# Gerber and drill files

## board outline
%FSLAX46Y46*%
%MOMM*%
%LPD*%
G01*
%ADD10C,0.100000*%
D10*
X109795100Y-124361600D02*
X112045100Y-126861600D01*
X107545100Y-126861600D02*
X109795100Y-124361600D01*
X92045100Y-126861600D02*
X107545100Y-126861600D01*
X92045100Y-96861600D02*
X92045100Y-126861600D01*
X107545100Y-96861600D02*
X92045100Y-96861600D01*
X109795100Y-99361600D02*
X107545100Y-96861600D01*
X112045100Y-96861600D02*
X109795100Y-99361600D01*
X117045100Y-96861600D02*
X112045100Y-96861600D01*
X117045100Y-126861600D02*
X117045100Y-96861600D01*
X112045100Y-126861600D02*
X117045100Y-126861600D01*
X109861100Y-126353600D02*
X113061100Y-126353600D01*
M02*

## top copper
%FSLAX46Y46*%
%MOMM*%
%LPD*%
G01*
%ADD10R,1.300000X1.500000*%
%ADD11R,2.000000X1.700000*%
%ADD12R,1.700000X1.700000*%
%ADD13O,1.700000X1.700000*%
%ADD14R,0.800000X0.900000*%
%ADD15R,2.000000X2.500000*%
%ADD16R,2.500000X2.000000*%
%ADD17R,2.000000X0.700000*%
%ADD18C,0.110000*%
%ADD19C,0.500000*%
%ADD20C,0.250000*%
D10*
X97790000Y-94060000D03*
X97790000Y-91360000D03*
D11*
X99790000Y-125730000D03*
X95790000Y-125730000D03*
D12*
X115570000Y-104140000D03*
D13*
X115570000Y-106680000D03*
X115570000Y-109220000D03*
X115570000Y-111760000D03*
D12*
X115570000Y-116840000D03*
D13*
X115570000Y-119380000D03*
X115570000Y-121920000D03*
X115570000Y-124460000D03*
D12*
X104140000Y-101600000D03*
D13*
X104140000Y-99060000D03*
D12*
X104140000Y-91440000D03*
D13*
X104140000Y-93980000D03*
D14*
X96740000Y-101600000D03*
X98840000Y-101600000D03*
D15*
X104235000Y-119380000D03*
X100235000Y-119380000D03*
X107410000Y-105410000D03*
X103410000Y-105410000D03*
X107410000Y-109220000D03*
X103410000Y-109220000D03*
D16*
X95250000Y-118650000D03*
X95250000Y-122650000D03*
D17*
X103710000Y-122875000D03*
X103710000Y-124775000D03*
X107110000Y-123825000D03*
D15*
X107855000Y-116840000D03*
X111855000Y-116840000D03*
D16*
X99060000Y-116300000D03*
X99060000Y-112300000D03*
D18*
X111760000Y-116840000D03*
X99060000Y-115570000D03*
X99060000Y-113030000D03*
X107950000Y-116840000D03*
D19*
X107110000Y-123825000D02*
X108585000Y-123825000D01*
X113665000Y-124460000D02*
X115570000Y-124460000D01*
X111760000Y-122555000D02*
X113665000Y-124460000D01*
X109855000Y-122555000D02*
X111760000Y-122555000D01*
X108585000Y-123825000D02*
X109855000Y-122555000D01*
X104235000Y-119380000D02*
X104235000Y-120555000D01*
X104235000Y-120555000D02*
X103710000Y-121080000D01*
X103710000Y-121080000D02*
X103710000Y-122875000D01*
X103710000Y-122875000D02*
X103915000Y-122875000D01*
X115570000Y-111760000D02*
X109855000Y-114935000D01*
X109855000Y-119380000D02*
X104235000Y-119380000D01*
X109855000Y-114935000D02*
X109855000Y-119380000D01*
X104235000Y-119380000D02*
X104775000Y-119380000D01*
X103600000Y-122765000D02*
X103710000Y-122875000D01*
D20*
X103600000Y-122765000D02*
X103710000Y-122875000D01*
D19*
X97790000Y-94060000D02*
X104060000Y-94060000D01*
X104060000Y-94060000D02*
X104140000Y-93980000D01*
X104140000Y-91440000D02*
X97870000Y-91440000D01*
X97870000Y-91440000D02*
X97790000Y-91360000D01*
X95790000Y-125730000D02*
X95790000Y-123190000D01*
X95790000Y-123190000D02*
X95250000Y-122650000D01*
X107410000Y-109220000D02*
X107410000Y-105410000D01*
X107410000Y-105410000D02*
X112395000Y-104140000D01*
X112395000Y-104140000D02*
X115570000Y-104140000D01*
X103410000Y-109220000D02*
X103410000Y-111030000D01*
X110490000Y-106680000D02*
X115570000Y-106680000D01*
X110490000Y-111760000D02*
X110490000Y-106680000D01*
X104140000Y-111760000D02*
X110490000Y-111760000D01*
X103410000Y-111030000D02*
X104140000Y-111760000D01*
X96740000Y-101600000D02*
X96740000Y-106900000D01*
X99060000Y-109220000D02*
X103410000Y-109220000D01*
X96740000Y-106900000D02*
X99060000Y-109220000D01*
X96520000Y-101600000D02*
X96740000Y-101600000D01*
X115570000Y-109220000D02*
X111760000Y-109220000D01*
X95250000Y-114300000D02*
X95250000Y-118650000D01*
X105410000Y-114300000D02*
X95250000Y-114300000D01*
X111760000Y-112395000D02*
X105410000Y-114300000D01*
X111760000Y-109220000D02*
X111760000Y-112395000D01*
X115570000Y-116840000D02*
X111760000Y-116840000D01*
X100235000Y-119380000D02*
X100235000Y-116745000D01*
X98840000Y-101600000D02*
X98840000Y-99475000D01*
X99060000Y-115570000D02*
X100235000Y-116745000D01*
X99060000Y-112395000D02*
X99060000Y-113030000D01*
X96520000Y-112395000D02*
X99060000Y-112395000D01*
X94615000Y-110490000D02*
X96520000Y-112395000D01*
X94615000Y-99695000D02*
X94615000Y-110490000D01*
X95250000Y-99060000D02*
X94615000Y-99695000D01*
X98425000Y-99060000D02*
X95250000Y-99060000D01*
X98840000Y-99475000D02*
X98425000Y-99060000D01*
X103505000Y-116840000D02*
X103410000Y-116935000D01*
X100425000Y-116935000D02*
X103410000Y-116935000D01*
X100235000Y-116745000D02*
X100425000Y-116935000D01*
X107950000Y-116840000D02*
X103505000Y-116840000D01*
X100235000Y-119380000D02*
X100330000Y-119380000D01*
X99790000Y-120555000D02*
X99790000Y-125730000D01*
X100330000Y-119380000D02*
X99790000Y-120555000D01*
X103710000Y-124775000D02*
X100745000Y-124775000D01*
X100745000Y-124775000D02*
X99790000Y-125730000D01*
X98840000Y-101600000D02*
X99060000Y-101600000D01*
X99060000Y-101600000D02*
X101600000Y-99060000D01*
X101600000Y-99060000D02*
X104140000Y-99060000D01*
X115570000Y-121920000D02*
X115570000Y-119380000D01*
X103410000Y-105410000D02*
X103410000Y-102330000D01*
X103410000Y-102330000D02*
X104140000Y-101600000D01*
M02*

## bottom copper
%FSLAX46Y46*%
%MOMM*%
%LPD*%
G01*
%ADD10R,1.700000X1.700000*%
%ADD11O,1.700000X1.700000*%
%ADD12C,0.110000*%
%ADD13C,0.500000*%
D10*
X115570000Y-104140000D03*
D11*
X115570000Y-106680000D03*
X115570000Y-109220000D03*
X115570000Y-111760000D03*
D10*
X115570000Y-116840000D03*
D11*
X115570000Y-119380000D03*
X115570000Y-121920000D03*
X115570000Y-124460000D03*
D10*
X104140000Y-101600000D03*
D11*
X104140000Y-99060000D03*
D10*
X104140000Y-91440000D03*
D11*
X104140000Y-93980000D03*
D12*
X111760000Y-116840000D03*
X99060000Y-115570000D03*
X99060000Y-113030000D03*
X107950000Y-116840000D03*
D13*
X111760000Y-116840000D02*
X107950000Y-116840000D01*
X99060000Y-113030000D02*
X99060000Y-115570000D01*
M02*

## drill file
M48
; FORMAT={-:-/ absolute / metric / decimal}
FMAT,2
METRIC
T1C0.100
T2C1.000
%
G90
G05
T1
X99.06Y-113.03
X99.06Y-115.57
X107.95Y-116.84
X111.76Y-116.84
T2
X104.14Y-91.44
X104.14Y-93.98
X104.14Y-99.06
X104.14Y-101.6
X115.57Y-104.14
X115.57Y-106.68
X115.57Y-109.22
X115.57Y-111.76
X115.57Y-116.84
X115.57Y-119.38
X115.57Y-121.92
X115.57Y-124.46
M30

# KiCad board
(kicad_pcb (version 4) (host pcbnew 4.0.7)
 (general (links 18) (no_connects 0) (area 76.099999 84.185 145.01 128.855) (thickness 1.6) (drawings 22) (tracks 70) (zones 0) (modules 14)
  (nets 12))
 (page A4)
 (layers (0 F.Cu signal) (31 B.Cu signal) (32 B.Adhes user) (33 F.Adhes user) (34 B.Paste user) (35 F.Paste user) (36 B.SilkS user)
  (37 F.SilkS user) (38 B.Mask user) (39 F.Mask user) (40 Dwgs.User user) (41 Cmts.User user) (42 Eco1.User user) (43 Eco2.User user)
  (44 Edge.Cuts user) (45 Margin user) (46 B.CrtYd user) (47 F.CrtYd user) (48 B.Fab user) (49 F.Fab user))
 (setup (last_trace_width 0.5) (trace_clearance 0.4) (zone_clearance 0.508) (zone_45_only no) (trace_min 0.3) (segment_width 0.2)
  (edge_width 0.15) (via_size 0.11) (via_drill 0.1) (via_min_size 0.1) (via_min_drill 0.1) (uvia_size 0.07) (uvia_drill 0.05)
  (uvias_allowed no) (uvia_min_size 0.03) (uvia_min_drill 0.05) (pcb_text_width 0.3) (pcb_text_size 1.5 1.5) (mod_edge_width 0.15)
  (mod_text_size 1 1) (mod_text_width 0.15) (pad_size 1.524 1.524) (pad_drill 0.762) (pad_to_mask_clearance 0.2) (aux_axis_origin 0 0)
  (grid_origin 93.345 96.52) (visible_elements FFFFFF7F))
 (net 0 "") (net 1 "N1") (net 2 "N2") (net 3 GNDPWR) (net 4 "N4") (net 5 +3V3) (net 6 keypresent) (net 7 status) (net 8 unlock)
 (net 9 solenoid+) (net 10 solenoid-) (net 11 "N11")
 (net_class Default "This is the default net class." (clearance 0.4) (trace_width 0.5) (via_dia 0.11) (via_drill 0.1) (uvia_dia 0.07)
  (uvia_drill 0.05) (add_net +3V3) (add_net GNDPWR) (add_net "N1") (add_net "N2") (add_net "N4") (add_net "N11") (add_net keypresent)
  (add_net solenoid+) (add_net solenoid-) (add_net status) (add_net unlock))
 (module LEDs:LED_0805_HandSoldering (layer F.Cu) (at 97.79 92.71 90)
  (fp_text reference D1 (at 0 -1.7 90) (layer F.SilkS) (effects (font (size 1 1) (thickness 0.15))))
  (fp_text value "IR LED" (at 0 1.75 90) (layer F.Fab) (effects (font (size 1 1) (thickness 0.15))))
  (pad 1 smd rect (at -1.35 0 90) (size 1.5 1.3) (layers F.Cu F.Paste F.Mask) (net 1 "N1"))
  (pad 2 smd rect (at 1.35 0 90) (size 1.5 1.3) (layers F.Cu F.Paste F.Mask) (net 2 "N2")))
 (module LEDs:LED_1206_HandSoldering (layer F.Cu) (at 97.79 125.73 180)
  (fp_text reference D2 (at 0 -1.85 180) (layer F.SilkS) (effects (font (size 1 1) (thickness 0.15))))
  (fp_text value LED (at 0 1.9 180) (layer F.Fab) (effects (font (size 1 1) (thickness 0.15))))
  (pad 1 smd rect (at -2 0 180) (size 2 1.7) (layers F.Cu F.Paste F.Mask) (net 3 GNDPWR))
  (pad 2 smd rect (at 2 0 180) (size 2 1.7) (layers F.Cu F.Paste F.Mask) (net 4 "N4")))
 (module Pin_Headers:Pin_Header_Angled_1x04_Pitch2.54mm (layer F.Cu) (at 115.57 104.14)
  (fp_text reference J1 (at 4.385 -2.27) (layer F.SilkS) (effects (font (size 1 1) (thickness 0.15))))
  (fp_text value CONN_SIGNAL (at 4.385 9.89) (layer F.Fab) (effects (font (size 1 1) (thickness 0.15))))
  (pad 1 thru_hole rect (at 0 0) (size 1.7 1.7) (drill 1) (layers *.Cu *.Mask) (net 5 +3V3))
  (pad 2 thru_hole oval (at 0 2.54) (size 1.7 1.7) (drill 1) (layers *.Cu *.Mask) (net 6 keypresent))
  (pad 3 thru_hole oval (at 0 5.08) (size 1.7 1.7) (drill 1) (layers *.Cu *.Mask) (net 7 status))
  (pad 4 thru_hole oval (at 0 7.62) (size 1.7 1.7) (drill 1) (layers *.Cu *.Mask) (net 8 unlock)))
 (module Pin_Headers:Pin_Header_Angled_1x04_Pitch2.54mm (layer F.Cu) (at 115.57 116.84)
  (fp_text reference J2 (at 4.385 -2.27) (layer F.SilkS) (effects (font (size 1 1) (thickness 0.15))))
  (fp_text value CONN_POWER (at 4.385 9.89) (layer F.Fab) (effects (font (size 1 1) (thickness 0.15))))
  (pad 1 thru_hole rect (at 0 0) (size 1.7 1.7) (drill 1) (layers *.Cu *.Mask) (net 3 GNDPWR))
  (pad 2 thru_hole oval (at 0 2.54) (size 1.7 1.7) (drill 1) (layers *.Cu *.Mask) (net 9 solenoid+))
  (pad 3 thru_hole oval (at 0 5.08) (size 1.7 1.7) (drill 1) (layers *.Cu *.Mask) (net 9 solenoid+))
  (pad 4 thru_hole oval (at 0 7.62) (size 1.7 1.7) (drill 1) (layers *.Cu *.Mask) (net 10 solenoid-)))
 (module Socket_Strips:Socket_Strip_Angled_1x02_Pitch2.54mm (layer F.Cu) (at 104.14 101.6 180)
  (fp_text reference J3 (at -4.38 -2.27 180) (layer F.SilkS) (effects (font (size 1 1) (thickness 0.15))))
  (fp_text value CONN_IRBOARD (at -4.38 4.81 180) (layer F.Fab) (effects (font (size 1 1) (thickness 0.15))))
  (pad 1 thru_hole rect (at 0 0 180) (size 1.7 1.7) (drill 1) (layers *.Cu *.Mask) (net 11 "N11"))
  (pad 2 thru_hole oval (at 0 2.54 180) (size 1.7 1.7) (drill 1) (layers *.Cu *.Mask) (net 3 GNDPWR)))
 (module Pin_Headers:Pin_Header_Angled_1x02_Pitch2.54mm (layer F.Cu) (at 104.14 91.44)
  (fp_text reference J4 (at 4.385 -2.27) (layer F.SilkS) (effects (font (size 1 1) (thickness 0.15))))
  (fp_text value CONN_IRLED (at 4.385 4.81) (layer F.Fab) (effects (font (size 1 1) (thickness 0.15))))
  (pad 1 thru_hole rect (at 0 0) (size 1.7 1.7) (drill 1) (layers *.Cu *.Mask) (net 2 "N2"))
  (pad 2 thru_hole oval (at 0 2.54) (size 1.7 1.7) (drill 1) (layers *.Cu *.Mask) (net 1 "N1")))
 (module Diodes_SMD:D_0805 (layer F.Cu) (at 97.79 101.6)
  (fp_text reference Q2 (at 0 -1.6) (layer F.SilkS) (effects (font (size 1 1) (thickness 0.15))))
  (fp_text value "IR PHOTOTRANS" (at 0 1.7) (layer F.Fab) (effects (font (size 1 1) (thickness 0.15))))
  (pad 1 smd rect (at -1.05 0) (size 0.8 0.9) (layers F.Cu F.Paste F.Mask) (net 6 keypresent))
  (pad 2 smd rect (at 1.05 0) (size 0.8 0.9) (layers F.Cu F.Paste F.Mask) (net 3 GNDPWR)))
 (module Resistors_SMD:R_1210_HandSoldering (layer F.Cu) (at 102.235 119.38 180)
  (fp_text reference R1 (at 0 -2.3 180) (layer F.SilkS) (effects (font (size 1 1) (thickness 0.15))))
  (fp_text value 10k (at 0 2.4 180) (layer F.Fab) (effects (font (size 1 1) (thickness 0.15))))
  (pad 1 smd rect (at -2 0 180) (size 2 2.5) (layers F.Cu F.Paste F.Mask) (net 8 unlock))
  (pad 2 smd rect (at 2 0 180) (size 2 2.5) (layers F.Cu F.Paste F.Mask) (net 3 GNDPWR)))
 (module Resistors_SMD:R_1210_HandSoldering (layer F.Cu) (at 105.41 105.41 180)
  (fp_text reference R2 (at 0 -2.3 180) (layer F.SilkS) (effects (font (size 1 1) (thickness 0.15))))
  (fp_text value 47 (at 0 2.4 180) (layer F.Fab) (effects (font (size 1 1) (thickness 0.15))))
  (pad 1 smd rect (at -2 0 180) (size 2 2.5) (layers F.Cu F.Paste F.Mask) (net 5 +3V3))
  (pad 2 smd rect (at 2 0 180) (size 2 2.5) (layers F.Cu F.Paste F.Mask) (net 11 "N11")))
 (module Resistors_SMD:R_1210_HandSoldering (layer F.Cu) (at 105.41 109.22 180)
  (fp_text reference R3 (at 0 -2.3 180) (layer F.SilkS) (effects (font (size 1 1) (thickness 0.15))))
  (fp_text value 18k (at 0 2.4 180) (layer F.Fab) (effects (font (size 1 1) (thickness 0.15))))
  (pad 1 smd rect (at -2 0 180) (size 2 2.5) (layers F.Cu F.Paste F.Mask) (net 5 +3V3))
  (pad 2 smd rect (at 2 0 180) (size 2 2.5) (layers F.Cu F.Paste F.Mask) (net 6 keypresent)))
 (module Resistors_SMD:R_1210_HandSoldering (layer F.Cu) (at 95.25 120.65 270)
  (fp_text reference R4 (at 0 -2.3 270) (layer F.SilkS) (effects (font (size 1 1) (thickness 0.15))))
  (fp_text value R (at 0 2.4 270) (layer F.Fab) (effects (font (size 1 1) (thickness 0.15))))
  (pad 1 smd rect (at -2 0 270) (size 2 2.5) (layers F.Cu F.Paste F.Mask) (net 7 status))
  (pad 2 smd rect (at 2 0 270) (size 2 2.5) (layers F.Cu F.Paste F.Mask) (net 4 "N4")))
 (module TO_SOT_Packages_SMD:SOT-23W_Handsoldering (layer F.Cu) (at 105.41 123.825)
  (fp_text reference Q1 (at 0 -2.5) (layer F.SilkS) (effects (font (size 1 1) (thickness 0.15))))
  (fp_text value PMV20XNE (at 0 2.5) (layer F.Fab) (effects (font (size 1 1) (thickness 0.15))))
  (pad 1 smd rect (at -1.7 -0.95) (size 2 0.7) (layers F.Cu F.Paste F.Mask) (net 8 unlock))
  (pad 2 smd rect (at -1.7 0.95) (size 2 0.7) (layers F.Cu F.Paste F.Mask) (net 3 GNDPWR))
  (pad 3 smd rect (at 1.7 0) (size 2 0.7) (layers F.Cu F.Paste F.Mask) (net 10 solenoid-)))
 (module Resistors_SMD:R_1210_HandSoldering (layer F.Cu) (at 109.855 116.84)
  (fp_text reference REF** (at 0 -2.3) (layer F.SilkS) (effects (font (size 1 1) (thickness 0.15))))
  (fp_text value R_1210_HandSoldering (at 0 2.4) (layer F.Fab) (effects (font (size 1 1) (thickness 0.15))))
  (pad 1 smd rect (at -2 0) (size 2 2.5) (layers F.Cu F.Paste F.Mask))
  (pad 2 smd rect (at 2 0) (size 2 2.5) (layers F.Cu F.Paste F.Mask)))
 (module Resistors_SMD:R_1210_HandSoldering (layer F.Cu) (at 99.06 114.3 90)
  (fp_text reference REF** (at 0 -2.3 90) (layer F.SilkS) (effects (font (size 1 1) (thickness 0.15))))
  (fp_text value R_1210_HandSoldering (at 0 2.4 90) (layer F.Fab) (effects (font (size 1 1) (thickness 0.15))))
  (pad 1 smd rect (at -2 0 90) (size 2 2.5) (layers F.Cu F.Paste F.Mask))
  (pad 2 smd rect (at 2 0 90) (size 2 2.5) (layers F.Cu F.Paste F.Mask)))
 (gr_line (start 109.7951 124.3616) (end 112.0451 126.8616) (layer Edge.Cuts) (width 0.1))
 (gr_line (start 107.5451 126.8616) (end 109.7951 124.3616) (layer Edge.Cuts) (width 0.1))
 (gr_line (start 92.0451 126.8616) (end 107.5451 126.8616) (layer Edge.Cuts) (width 0.1))
 (gr_line (start 92.0451 96.8616) (end 92.0451 126.8616) (layer Edge.Cuts) (width 0.1))
 (gr_line (start 107.5451 96.8616) (end 92.0451 96.8616) (layer Edge.Cuts) (width 0.1))
 (gr_line (start 109.7951 99.3616) (end 107.5451 96.8616) (layer Edge.Cuts) (width 0.1))
 (gr_line (start 112.0451 96.8616) (end 109.7951 99.3616) (layer Edge.Cuts) (width 0.1))
 (gr_line (start 117.0451 96.8616) (end 112.0451 96.8616) (layer Edge.Cuts) (width 0.1))
 (gr_line (start 117.0451 126.8616) (end 117.0451 96.8616) (layer Edge.Cuts) (width 0.1))
 (gr_line (start 112.0451 126.8616) (end 117.0451 126.8616) (layer Edge.Cuts) (width 0.1))
 (gr_line (start 109.8611 126.3536) (end 113.0611 126.3536) (layer Edge.Cuts) (width 0.1))
 (segment (start 107.11 123.825) (end 108.585 123.825) (width 0.5) (layer F.Cu) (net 10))
 (segment (start 113.665 124.46) (end 115.57 124.46) (width 0.5) (layer F.Cu) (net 10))
 (segment (start 111.76 122.555) (end 113.665 124.46) (width 0.5) (layer F.Cu) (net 10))
 (segment (start 109.855 122.555) (end 111.76 122.555) (width 0.5) (layer F.Cu) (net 10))
 (segment (start 108.585 123.825) (end 109.855 122.555) (width 0.5) (layer F.Cu) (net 10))
 (segment (start 104.235 119.38) (end 104.235 120.555) (width 0.5) (layer F.Cu) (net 8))
 (segment (start 104.235 120.555) (end 103.71 121.08) (width 0.5) (layer F.Cu) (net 8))
 (segment (start 103.71 121.08) (end 103.71 122.875) (width 0.5) (layer F.Cu) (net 8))
 (segment (start 103.71 122.875) (end 103.915 122.875) (width 0.5) (layer F.Cu) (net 8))
 (segment (start 115.57 111.76) (end 109.855 114.935) (width 0.5) (layer F.Cu) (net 8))
 (segment (start 109.855 119.38) (end 104.235 119.38) (width 0.5) (layer F.Cu) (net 8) (status 20))
 (segment (start 109.855 114.935) (end 109.855 119.38) (width 0.5) (layer F.Cu) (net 8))
 (segment (start 104.235 119.38) (end 104.775 119.38) (width 0.5) (layer F.Cu) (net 8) (status 30))
 (segment (start 103.6 122.765) (end 103.71 122.875) (width 0.5) (layer F.Cu) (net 8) (status 30))
 (segment (start 103.6 122.765) (end 103.71 122.875) (width 0.25) (layer F.Cu) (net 8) (status 30))
 (segment (start 97.79 94.06) (end 104.06 94.06) (width 0.5) (layer F.Cu) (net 1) (status 10))
 (segment (start 104.06 94.06) (end 104.14 93.98) (width 0.5) (layer F.Cu) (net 1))
 (segment (start 104.14 91.44) (end 97.87 91.44) (width 0.5) (layer F.Cu) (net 2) (status 20))
 (segment (start 97.87 91.44) (end 97.79 91.36) (width 0.5) (layer F.Cu) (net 2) (status 30))
 (segment (start 95.79 125.73) (end 95.79 123.19) (width 0.5) (layer F.Cu) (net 4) (status 10))
 (segment (start 95.79 123.19) (end 95.25 122.65) (width 0.5) (layer F.Cu) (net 4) (status 30))
 (segment (start 107.41 109.22) (end 107.41 105.41) (width 0.5) (layer F.Cu) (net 5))
 (segment (start 107.41 105.41) (end 112.395 104.14) (width 0.5) (layer F.Cu) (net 5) (status 10))
 (segment (start 112.395 104.14) (end 115.57 104.14) (width 0.5) (layer F.Cu) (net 5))
 (segment (start 103.41 109.22) (end 103.41 111.03) (width 0.5) (layer F.Cu) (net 6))
 (segment (start 110.49 106.68) (end 115.57 106.68) (width 0.5) (layer F.Cu) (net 6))
 (segment (start 110.49 111.76) (end 110.49 106.68) (width 0.5) (layer F.Cu) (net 6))
 (segment (start 104.14 111.76) (end 110.49 111.76) (width 0.5) (layer F.Cu) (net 6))
 (segment (start 103.41 111.03) (end 104.14 111.76) (width 0.5) (layer F.Cu) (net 6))
 (segment (start 96.74 101.6) (end 96.74 106.9) (width 0.5) (layer F.Cu) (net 6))
 (segment (start 99.06 109.22) (end 103.41 109.22) (width 0.5) (layer F.Cu) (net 6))
 (segment (start 96.74 106.9) (end 99.06 109.22) (width 0.5) (layer F.Cu) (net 6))
 (segment (start 96.52 101.6) (end 96.74 101.6) (width 0.5) (layer F.Cu) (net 6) (status 30))
 (segment (start 115.57 109.22) (end 111.76 109.22) (width 0.5) (layer F.Cu) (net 7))
 (segment (start 95.25 114.3) (end 95.25 118.65) (width 0.5) (layer F.Cu) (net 7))
 (segment (start 105.41 114.3) (end 95.25 114.3) (width 0.5) (layer F.Cu) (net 7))
 (segment (start 111.76 112.395) (end 105.41 114.3) (width 0.5) (layer F.Cu) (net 7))
 (segment (start 111.76 109.22) (end 111.76 112.395) (width 0.5) (layer F.Cu) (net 7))
 (segment (start 115.57 116.84) (end 111.76 116.84) (width 0.5) (layer F.Cu) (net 3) (status 20))
 (via (at 111.76 116.84) (size 0.11) (drill 0.1) (layers F.Cu B.Cu) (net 3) (status 30))
 (segment (start 111.76 116.84) (end 107.95 116.84) (width 0.5) (layer B.Cu) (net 3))
 (segment (start 100.235 119.38) (end 100.235 116.745) (width 0.5) (layer F.Cu) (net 3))
 (segment (start 98.84 101.6) (end 98.84 99.475) (width 0.5) (layer F.Cu) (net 3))
 (segment (start 99.06 115.57) (end 100.235 116.745) (width 0.5) (layer F.Cu) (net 3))
 (via (at 99.06 115.57) (size 0.11) (drill 0.1) (layers F.Cu B.Cu) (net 3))
 (segment (start 99.06 113.03) (end 99.06 115.57) (width 0.5) (layer B.Cu) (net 3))
 (via (at 99.06 113.03) (size 0.11) (drill 0.1) (layers F.Cu B.Cu) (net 3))
 (segment (start 99.06 112.395) (end 99.06 113.03) (width 0.5) (layer F.Cu) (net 3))
 (segment (start 96.52 112.395) (end 99.06 112.395) (width 0.5) (layer F.Cu) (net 3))
 (segment (start 94.615 110.49) (end 96.52 112.395) (width 0.5) (layer F.Cu) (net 3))
 (segment (start 94.615 99.695) (end 94.615 110.49) (width 0.5) (layer F.Cu) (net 3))
 (segment (start 95.25 99.06) (end 94.615 99.695) (width 0.5) (layer F.Cu) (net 3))
 (segment (start 98.425 99.06) (end 95.25 99.06) (width 0.5) (layer F.Cu) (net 3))
 (segment (start 98.84 99.475) (end 98.425 99.06) (width 0.5) (layer F.Cu) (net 3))
 (segment (start 103.505 116.84) (end 103.41 116.935) (width 0.5) (layer F.Cu) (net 3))
 (segment (start 100.425 116.935) (end 103.41 116.935) (width 0.5) (layer F.Cu) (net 3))
 (segment (start 100.235 116.745) (end 100.425 116.935) (width 0.5) (layer F.Cu) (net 3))
 (via (at 107.95 116.84) (size 0.11) (drill 0.1) (layers F.Cu B.Cu) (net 3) (status 30))
 (segment (start 107.95 116.84) (end 103.505 116.84) (width 0.5) (layer F.Cu) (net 3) (status 10))
 (segment (start 100.235 119.38) (end 100.33 119.38) (width 0.5) (layer F.Cu) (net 3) (status 30))
 (segment (start 99.79 120.555) (end 99.79 125.73) (width 0.5) (layer F.Cu) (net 3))
 (segment (start 100.33 119.38) (end 99.79 120.555) (width 0.5) (layer F.Cu) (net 3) (status 10))
 (segment (start 103.71 124.775) (end 100.745 124.775) (width 0.5) (layer F.Cu) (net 3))
 (segment (start 100.745 124.775) (end 99.79 125.73) (width 0.5) (layer F.Cu) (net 3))
 (segment (start 98.84 101.6) (end 99.06 101.6) (width 0.5) (layer F.Cu) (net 3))
 (segment (start 99.06 101.6) (end 101.6 99.06) (width 0.5) (layer F.Cu) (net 3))
 (segment (start 101.6 99.06) (end 104.14 99.06) (width 0.5) (layer F.Cu) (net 3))
 (segment (start 115.57 121.92) (end 115.57 119.38) (width 0.5) (layer F.Cu) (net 9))
 (segment (start 103.41 105.41) (end 103.41 102.33) (width 0.5) (layer F.Cu) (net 11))
 (segment (start 103.41 102.33) (end 104.14 101.6) (width 0.5) (layer F.Cu) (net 11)))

